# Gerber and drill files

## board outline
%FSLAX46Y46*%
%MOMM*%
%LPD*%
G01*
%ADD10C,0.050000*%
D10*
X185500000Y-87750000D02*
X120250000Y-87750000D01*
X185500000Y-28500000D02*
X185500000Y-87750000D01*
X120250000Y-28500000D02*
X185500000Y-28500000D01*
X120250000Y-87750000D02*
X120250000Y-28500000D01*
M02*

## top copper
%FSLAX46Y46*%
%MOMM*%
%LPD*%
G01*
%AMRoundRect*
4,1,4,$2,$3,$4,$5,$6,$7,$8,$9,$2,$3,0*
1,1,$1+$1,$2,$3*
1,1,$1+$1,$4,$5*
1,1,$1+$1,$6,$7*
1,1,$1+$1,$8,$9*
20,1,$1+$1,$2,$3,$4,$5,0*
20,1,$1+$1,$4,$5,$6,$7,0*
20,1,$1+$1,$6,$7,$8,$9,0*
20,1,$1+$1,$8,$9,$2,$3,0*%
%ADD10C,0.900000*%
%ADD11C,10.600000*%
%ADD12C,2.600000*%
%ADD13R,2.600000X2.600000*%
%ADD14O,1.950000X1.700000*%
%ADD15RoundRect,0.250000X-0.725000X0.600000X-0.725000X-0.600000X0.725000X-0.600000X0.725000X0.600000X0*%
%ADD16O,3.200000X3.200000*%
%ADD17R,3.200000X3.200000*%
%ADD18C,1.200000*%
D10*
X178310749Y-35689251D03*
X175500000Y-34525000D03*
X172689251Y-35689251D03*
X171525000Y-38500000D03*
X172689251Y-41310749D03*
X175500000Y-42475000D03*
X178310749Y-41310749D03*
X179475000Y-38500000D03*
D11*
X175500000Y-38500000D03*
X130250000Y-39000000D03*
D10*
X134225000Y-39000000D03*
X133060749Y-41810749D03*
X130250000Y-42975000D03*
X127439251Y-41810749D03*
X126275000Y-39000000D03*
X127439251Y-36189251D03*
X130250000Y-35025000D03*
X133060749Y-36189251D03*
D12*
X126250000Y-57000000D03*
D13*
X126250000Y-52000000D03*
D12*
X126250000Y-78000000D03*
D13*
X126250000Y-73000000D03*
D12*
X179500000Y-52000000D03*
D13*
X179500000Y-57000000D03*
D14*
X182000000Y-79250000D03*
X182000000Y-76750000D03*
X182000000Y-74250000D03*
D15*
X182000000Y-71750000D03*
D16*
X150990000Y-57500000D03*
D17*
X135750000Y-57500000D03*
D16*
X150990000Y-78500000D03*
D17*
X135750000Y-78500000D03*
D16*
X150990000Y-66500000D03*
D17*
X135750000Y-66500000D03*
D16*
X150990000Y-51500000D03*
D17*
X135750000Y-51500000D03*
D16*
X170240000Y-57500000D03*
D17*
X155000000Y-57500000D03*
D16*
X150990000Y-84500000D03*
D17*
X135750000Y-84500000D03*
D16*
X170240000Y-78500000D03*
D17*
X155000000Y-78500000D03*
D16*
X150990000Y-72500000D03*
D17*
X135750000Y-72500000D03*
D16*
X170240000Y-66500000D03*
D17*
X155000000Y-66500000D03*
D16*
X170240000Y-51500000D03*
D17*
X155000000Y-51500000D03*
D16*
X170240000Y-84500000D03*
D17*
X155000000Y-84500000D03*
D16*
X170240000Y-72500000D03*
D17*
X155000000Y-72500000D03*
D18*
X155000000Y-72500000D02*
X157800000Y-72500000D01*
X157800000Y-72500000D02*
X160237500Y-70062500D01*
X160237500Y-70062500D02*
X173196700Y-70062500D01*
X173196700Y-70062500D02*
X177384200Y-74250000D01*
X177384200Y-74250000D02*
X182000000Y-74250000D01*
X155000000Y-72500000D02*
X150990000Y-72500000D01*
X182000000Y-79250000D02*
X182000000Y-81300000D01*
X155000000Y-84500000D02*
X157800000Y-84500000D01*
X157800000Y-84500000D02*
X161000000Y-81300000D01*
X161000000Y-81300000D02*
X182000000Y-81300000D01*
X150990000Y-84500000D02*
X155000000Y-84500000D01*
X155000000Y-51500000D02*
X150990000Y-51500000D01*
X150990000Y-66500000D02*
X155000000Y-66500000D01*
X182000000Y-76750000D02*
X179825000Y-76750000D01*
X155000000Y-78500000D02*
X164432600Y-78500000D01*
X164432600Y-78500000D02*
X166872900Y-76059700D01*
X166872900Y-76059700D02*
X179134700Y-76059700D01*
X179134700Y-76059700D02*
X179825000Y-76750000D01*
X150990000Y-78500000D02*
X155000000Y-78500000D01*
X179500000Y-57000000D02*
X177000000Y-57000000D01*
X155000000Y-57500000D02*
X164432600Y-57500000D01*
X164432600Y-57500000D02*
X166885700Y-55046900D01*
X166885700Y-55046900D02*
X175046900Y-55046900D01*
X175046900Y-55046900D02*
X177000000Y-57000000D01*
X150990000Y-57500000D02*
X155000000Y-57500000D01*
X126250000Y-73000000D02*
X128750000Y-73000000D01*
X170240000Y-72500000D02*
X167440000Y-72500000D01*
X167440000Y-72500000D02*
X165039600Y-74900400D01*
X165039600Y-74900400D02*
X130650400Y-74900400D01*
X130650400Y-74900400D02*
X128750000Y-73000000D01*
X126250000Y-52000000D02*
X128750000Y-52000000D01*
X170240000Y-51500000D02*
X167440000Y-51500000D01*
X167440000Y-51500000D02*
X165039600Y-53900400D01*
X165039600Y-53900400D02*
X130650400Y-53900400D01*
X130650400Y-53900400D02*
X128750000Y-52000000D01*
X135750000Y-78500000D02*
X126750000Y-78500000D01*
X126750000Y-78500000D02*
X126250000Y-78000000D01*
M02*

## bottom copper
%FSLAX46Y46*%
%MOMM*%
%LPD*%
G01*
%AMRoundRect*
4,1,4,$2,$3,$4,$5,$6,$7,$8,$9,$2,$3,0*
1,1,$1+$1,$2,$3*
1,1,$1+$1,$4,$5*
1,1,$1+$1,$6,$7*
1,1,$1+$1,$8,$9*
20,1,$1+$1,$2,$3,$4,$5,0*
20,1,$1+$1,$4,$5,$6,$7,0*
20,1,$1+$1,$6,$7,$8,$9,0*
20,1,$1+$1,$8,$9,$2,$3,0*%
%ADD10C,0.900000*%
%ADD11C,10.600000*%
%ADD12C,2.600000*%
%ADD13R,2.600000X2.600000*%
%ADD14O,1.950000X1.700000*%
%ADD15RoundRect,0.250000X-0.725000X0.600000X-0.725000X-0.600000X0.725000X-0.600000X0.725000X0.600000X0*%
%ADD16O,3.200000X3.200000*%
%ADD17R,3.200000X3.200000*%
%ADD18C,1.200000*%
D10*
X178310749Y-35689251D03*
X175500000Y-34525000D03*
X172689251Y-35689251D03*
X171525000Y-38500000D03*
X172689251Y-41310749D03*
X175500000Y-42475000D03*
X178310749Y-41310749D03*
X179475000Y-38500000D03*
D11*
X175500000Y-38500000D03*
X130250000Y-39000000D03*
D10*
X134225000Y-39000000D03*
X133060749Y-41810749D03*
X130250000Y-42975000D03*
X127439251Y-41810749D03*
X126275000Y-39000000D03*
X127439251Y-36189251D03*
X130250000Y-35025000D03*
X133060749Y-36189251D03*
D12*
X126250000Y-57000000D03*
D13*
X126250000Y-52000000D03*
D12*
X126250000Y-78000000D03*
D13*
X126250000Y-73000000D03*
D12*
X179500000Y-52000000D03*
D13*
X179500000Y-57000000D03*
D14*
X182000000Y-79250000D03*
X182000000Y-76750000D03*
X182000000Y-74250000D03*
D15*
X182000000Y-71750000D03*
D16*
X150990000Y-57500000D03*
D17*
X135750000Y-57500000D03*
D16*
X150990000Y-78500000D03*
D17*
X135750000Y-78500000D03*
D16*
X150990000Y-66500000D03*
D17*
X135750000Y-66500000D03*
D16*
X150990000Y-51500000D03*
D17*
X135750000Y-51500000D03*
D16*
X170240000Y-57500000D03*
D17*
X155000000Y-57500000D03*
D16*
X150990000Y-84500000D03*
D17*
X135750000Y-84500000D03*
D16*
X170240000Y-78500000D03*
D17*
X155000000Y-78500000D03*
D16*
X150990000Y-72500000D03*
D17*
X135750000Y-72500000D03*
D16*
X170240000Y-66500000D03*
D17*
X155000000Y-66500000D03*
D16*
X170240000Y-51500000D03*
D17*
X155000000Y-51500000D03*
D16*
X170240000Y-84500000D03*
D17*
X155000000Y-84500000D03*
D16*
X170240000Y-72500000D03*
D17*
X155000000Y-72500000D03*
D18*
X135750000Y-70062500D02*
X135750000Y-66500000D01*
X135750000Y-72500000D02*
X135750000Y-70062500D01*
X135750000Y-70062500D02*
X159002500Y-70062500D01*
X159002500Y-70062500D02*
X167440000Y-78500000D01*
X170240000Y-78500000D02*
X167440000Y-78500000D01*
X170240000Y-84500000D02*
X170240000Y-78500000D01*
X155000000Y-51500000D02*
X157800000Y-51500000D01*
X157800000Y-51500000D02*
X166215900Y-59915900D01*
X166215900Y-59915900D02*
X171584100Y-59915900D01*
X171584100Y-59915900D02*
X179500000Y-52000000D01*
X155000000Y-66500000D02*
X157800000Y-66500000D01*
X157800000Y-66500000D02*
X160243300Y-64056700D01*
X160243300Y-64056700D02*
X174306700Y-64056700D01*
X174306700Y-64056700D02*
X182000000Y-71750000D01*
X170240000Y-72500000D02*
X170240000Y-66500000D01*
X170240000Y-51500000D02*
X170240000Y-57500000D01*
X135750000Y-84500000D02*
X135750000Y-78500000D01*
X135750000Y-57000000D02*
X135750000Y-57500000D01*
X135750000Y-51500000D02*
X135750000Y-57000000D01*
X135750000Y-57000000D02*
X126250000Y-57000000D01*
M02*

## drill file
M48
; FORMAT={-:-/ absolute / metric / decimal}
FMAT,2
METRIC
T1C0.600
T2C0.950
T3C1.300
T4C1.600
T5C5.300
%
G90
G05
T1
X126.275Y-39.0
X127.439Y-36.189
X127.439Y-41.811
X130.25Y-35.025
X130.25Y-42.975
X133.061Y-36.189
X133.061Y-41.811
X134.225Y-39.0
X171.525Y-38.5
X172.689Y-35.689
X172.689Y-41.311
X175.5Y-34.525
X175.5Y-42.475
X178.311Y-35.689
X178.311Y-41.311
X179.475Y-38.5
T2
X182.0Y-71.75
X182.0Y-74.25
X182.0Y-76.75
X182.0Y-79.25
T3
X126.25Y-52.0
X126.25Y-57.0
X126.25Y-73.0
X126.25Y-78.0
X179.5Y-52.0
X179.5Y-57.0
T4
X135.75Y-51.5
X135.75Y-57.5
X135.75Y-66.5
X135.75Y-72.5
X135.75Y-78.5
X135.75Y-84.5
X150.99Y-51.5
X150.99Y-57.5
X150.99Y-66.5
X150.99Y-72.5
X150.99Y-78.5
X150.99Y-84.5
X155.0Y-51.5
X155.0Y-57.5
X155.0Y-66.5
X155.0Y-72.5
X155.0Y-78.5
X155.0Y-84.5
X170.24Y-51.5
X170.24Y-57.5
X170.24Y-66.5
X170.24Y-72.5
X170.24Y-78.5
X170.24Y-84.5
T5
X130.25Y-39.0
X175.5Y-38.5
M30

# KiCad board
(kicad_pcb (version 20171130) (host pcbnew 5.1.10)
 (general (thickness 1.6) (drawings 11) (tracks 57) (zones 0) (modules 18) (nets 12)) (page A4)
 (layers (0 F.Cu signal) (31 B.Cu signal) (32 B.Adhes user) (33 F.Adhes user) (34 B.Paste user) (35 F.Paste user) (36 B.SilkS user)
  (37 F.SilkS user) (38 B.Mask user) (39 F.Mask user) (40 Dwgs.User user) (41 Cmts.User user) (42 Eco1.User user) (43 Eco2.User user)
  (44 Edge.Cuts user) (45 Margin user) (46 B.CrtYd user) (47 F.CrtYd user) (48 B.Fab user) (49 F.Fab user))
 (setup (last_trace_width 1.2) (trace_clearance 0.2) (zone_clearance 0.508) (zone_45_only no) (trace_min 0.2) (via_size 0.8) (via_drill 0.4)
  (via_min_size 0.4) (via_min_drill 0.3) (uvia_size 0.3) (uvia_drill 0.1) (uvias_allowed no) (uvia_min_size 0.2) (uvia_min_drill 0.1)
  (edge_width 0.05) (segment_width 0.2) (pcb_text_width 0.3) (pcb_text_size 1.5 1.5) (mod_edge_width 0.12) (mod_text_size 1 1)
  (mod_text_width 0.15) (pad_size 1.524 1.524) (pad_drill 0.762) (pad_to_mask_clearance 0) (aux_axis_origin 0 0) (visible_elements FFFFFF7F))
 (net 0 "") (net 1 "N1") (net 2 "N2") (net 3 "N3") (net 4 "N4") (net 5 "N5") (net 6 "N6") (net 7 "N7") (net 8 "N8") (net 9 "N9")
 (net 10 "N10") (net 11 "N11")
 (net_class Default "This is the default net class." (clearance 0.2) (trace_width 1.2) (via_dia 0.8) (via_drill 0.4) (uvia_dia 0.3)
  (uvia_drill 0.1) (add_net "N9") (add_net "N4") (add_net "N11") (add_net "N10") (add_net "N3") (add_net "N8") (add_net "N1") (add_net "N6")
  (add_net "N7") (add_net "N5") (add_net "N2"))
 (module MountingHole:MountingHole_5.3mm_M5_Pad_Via (layer F.Cu) (at 175.5 38.5)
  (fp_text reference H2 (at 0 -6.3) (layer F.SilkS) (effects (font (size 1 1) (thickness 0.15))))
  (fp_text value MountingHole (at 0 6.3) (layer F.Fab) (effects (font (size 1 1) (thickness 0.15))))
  (pad 1 thru_hole circle (at 2.810749 -2.810749) (size 0.9 0.9) (drill 0.6) (layers *.Cu *.Mask))
  (pad 1 thru_hole circle (at 0 -3.975) (size 0.9 0.9) (drill 0.6) (layers *.Cu *.Mask))
  (pad 1 thru_hole circle (at -2.810749 -2.810749) (size 0.9 0.9) (drill 0.6) (layers *.Cu *.Mask))
  (pad 1 thru_hole circle (at -3.975 0) (size 0.9 0.9) (drill 0.6) (layers *.Cu *.Mask))
  (pad 1 thru_hole circle (at -2.810749 2.810749) (size 0.9 0.9) (drill 0.6) (layers *.Cu *.Mask))
  (pad 1 thru_hole circle (at 0 3.975) (size 0.9 0.9) (drill 0.6) (layers *.Cu *.Mask))
  (pad 1 thru_hole circle (at 2.810749 2.810749) (size 0.9 0.9) (drill 0.6) (layers *.Cu *.Mask))
  (pad 1 thru_hole circle (at 3.975 0) (size 0.9 0.9) (drill 0.6) (layers *.Cu *.Mask))
  (pad 1 thru_hole circle (at 0 0) (size 10.6 10.6) (drill 5.3) (layers *.Cu *.Mask)))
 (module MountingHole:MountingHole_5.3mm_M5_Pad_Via (layer F.Cu) (at 130.25 39)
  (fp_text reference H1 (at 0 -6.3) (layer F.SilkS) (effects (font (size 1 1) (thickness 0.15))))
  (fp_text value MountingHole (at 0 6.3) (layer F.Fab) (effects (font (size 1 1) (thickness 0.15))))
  (pad 1 thru_hole circle (at 0 0) (size 10.6 10.6) (drill 5.3) (layers *.Cu *.Mask))
  (pad 1 thru_hole circle (at 3.975 0) (size 0.9 0.9) (drill 0.6) (layers *.Cu *.Mask))
  (pad 1 thru_hole circle (at 2.810749 2.810749) (size 0.9 0.9) (drill 0.6) (layers *.Cu *.Mask))
  (pad 1 thru_hole circle (at 0 3.975) (size 0.9 0.9) (drill 0.6) (layers *.Cu *.Mask))
  (pad 1 thru_hole circle (at -2.810749 2.810749) (size 0.9 0.9) (drill 0.6) (layers *.Cu *.Mask))
  (pad 1 thru_hole circle (at -3.975 0) (size 0.9 0.9) (drill 0.6) (layers *.Cu *.Mask))
  (pad 1 thru_hole circle (at -2.810749 -2.810749) (size 0.9 0.9) (drill 0.6) (layers *.Cu *.Mask))
  (pad 1 thru_hole circle (at 0 -3.975) (size 0.9 0.9) (drill 0.6) (layers *.Cu *.Mask))
  (pad 1 thru_hole circle (at 2.810749 -2.810749) (size 0.9 0.9) (drill 0.6) (layers *.Cu *.Mask)))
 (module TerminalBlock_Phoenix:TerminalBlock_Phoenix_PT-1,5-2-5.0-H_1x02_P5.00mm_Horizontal (layer F.Cu) (at 126.25 52 270)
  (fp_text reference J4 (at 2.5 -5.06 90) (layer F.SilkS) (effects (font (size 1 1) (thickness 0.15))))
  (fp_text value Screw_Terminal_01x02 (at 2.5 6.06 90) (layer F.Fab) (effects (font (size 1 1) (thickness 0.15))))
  (pad 2 thru_hole circle (at 5 0 270) (size 2.6 2.6) (drill 1.3) (layers *.Cu *.Mask) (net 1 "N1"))
  (pad 1 thru_hole rect (at 0 0 270) (size 2.6 2.6) (drill 1.3) (layers *.Cu *.Mask) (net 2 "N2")))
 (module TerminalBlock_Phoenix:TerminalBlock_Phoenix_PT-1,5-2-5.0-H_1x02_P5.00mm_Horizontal (layer F.Cu) (at 126.25 73 270)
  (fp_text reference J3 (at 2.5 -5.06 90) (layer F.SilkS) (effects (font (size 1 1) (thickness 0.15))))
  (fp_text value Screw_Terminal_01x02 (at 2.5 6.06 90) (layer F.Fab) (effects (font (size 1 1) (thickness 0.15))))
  (pad 2 thru_hole circle (at 5 0 270) (size 2.6 2.6) (drill 1.3) (layers *.Cu *.Mask) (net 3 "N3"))
  (pad 1 thru_hole rect (at 0 0 270) (size 2.6 2.6) (drill 1.3) (layers *.Cu *.Mask) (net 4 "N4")))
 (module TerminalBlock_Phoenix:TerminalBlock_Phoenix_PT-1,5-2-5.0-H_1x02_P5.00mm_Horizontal (layer F.Cu) (at 179.5 57 90)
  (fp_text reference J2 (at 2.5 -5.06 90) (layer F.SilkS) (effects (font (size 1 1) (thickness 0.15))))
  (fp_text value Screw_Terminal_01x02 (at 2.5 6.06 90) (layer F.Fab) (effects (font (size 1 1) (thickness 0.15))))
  (pad 2 thru_hole circle (at 5 0 90) (size 2.6 2.6) (drill 1.3) (layers *.Cu *.Mask) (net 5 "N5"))
  (pad 1 thru_hole rect (at 0 0 90) (size 2.6 2.6) (drill 1.3) (layers *.Cu *.Mask) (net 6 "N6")))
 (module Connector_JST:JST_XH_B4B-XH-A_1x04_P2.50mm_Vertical (layer F.Cu) (at 182 71.75 270)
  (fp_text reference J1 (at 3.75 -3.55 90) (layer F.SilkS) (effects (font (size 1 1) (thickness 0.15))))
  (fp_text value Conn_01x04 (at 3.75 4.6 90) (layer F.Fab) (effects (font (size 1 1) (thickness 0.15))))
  (pad 4 thru_hole oval (at 7.5 0 270) (size 1.7 1.95) (drill 0.95) (layers *.Cu *.Mask) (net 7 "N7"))
  (pad 3 thru_hole oval (at 5 0 270) (size 1.7 1.95) (drill 0.95) (layers *.Cu *.Mask) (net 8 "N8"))
  (pad 2 thru_hole oval (at 2.5 0 270) (size 1.7 1.95) (drill 0.95) (layers *.Cu *.Mask) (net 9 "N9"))
  (pad 1 thru_hole roundrect (at 0 0 270) (size 1.7 1.95) (drill 0.95) (layers *.Cu *.Mask) (roundrect_rratio 0.1470588235294118)
   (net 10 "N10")))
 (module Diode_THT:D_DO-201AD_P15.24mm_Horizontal (layer F.Cu) (at 135.75 57.5)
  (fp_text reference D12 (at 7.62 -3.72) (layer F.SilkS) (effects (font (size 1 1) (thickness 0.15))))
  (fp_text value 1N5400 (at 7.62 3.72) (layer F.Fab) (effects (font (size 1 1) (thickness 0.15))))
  (pad 2 thru_hole oval (at 15.24 0) (size 3.2 3.2) (drill 1.6) (layers *.Cu *.Mask) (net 6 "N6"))
  (pad 1 thru_hole rect (at 0 0) (size 3.2 3.2) (drill 1.6) (layers *.Cu *.Mask) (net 1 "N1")))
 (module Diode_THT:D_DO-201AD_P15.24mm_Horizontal (layer F.Cu) (at 135.75 78.5)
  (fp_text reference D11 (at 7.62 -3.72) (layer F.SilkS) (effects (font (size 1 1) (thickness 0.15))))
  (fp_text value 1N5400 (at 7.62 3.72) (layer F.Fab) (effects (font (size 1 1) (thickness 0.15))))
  (pad 2 thru_hole oval (at 15.24 0) (size 3.2 3.2) (drill 1.6) (layers *.Cu *.Mask) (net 8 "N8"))
  (pad 1 thru_hole rect (at 0 0) (size 3.2 3.2) (drill 1.6) (layers *.Cu *.Mask) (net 3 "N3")))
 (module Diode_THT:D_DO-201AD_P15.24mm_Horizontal (layer F.Cu) (at 135.75 66.5)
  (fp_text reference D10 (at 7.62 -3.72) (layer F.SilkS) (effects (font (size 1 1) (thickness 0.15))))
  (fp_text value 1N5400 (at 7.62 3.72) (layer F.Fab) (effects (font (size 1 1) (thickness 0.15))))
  (pad 2 thru_hole oval (at 15.24 0) (size 3.2 3.2) (drill 1.6) (layers *.Cu *.Mask) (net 10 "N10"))
  (pad 1 thru_hole rect (at 0 0) (size 3.2 3.2) (drill 1.6) (layers *.Cu *.Mask) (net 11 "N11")))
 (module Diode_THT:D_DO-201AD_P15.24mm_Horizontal (layer F.Cu) (at 135.75 51.5)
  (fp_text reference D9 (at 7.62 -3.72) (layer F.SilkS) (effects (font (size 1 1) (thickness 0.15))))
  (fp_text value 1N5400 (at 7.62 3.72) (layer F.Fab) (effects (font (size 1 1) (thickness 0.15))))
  (pad 2 thru_hole oval (at 15.24 0) (size 3.2 3.2) (drill 1.6) (layers *.Cu *.Mask) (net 5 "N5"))
  (pad 1 thru_hole rect (at 0 0) (size 3.2 3.2) (drill 1.6) (layers *.Cu *.Mask) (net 1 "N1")))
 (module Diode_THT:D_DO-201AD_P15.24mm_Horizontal (layer F.Cu) (at 155 57.5)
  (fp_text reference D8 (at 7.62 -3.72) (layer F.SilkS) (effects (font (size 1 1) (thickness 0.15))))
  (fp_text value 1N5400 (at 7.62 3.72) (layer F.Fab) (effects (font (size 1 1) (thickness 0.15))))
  (pad 2 thru_hole oval (at 15.24 0) (size 3.2 3.2) (drill 1.6) (layers *.Cu *.Mask) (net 2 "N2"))
  (pad 1 thru_hole rect (at 0 0) (size 3.2 3.2) (drill 1.6) (layers *.Cu *.Mask) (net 6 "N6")))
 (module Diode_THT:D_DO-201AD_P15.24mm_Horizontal (layer F.Cu) (at 135.75 84.5)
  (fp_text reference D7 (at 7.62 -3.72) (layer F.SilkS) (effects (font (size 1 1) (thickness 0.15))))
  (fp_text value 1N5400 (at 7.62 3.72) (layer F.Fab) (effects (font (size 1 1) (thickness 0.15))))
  (pad 2 thru_hole oval (at 15.24 0) (size 3.2 3.2) (drill 1.6) (layers *.Cu *.Mask) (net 7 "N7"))
  (pad 1 thru_hole rect (at 0 0) (size 3.2 3.2) (drill 1.6) (layers *.Cu *.Mask) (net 3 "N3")))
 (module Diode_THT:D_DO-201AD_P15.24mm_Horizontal (layer F.Cu) (at 155 78.5)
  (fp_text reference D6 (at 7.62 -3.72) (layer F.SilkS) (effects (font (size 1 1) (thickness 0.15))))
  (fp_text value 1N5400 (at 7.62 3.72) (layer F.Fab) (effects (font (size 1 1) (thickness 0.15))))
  (pad 2 thru_hole oval (at 15.24 0) (size 3.2 3.2) (drill 1.6) (layers *.Cu *.Mask) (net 11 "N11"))
  (pad 1 thru_hole rect (at 0 0) (size 3.2 3.2) (drill 1.6) (layers *.Cu *.Mask) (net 8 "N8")))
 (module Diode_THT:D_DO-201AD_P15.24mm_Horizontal (layer F.Cu) (at 135.75 72.5)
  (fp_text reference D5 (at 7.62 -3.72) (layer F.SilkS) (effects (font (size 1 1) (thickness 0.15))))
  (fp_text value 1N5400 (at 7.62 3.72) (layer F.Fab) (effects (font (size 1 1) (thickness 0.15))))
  (pad 2 thru_hole oval (at 15.24 0) (size 3.2 3.2) (drill 1.6) (layers *.Cu *.Mask) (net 9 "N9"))
  (pad 1 thru_hole rect (at 0 0) (size 3.2 3.2) (drill 1.6) (layers *.Cu *.Mask) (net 11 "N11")))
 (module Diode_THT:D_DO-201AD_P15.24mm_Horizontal (layer F.Cu) (at 155 66.5)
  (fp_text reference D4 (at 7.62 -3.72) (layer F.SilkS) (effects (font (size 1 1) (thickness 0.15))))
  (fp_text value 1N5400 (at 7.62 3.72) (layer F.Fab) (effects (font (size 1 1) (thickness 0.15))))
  (pad 2 thru_hole oval (at 15.24 0) (size 3.2 3.2) (drill 1.6) (layers *.Cu *.Mask) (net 4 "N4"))
  (pad 1 thru_hole rect (at 0 0) (size 3.2 3.2) (drill 1.6) (layers *.Cu *.Mask) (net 10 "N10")))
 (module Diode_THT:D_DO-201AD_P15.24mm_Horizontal (layer F.Cu) (at 155 51.5)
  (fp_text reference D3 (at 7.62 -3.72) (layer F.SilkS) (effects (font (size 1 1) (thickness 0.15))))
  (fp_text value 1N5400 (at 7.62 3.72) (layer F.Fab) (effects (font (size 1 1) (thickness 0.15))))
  (pad 2 thru_hole oval (at 15.24 0) (size 3.2 3.2) (drill 1.6) (layers *.Cu *.Mask) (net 2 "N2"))
  (pad 1 thru_hole rect (at 0 0) (size 3.2 3.2) (drill 1.6) (layers *.Cu *.Mask) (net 5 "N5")))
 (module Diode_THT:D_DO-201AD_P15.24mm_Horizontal (layer F.Cu) (at 155 84.5)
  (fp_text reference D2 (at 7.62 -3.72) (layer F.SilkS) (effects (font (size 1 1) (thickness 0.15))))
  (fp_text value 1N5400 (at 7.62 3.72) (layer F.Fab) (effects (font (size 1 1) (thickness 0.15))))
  (pad 2 thru_hole oval (at 15.24 0) (size 3.2 3.2) (drill 1.6) (layers *.Cu *.Mask) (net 11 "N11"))
  (pad 1 thru_hole rect (at 0 0) (size 3.2 3.2) (drill 1.6) (layers *.Cu *.Mask) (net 7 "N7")))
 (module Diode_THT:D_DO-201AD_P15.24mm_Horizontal (layer F.Cu) (at 155 72.5)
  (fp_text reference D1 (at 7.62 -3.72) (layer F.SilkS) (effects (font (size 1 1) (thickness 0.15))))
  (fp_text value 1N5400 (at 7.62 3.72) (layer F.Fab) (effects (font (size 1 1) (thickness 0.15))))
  (pad 2 thru_hole oval (at 15.24 0) (size 3.2 3.2) (drill 1.6) (layers *.Cu *.Mask) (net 4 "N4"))
  (pad 1 thru_hole rect (at 0 0) (size 3.2 3.2) (drill 1.6) (layers *.Cu *.Mask) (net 9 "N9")))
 (gr_line (start 185.5 87.75) (end 120.25 87.75) (layer Edge.Cuts) (width 0.05))
 (gr_line (start 185.5 28.5) (end 185.5 87.75) (layer Edge.Cuts) (width 0.05))
 (gr_line (start 120.25 28.5) (end 185.5 28.5) (layer Edge.Cuts) (width 0.05))
 (gr_line (start 120.25 87.75) (end 120.25 28.5) (layer Edge.Cuts) (width 0.05))
 (segment (start 155 72.5) (end 157.8 72.5) (width 1.2) (layer F.Cu) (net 9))
 (segment (start 157.8 72.5) (end 160.2375 70.0625) (width 1.2) (layer F.Cu) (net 9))
 (segment (start 160.2375 70.0625) (end 173.1967 70.0625) (width 1.2) (layer F.Cu) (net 9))
 (segment (start 173.1967 70.0625) (end 177.3842 74.25) (width 1.2) (layer F.Cu) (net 9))
 (segment (start 177.3842 74.25) (end 182 74.25) (width 1.2) (layer F.Cu) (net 9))
 (segment (start 155 72.5) (end 150.99 72.5) (width 1.2) (layer F.Cu) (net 9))
 (segment (start 135.75 70.0625) (end 135.75 66.5) (width 1.2) (layer B.Cu) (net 11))
 (segment (start 135.75 72.5) (end 135.75 70.0625) (width 1.2) (layer B.Cu) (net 11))
 (segment (start 135.75 70.0625) (end 159.0025 70.0625) (width 1.2) (layer B.Cu) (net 11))
 (segment (start 159.0025 70.0625) (end 167.44 78.5) (width 1.2) (layer B.Cu) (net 11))
 (segment (start 170.24 78.5) (end 167.44 78.5) (width 1.2) (layer B.Cu) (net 11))
 (segment (start 170.24 84.5) (end 170.24 78.5) (width 1.2) (layer B.Cu) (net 11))
 (segment (start 182 79.25) (end 182 81.3) (width 1.2) (layer F.Cu) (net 7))
 (segment (start 155 84.5) (end 157.8 84.5) (width 1.2) (layer F.Cu) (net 7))
 (segment (start 157.8 84.5) (end 161 81.3) (width 1.2) (layer F.Cu) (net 7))
 (segment (start 161 81.3) (end 182 81.3) (width 1.2) (layer F.Cu) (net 7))
 (segment (start 150.99 84.5) (end 155 84.5) (width 1.2) (layer F.Cu) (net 7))
 (segment (start 155 51.5) (end 157.8 51.5) (width 1.2) (layer B.Cu) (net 5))
 (segment (start 157.8 51.5) (end 166.2159 59.9159) (width 1.2) (layer B.Cu) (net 5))
 (segment (start 166.2159 59.9159) (end 171.5841 59.9159) (width 1.2) (layer B.Cu) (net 5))
 (segment (start 171.5841 59.9159) (end 179.5 52) (width 1.2) (layer B.Cu) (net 5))
 (segment (start 155 51.5) (end 150.99 51.5) (width 1.2) (layer F.Cu) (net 5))
 (segment (start 155 66.5) (end 157.8 66.5) (width 1.2) (layer B.Cu) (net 10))
 (segment (start 157.8 66.5) (end 160.2433 64.0567) (width 1.2) (layer B.Cu) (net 10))
 (segment (start 160.2433 64.0567) (end 174.3067 64.0567) (width 1.2) (layer B.Cu) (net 10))
 (segment (start 174.3067 64.0567) (end 182 71.75) (width 1.2) (layer B.Cu) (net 10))
 (segment (start 150.99 66.5) (end 155 66.5) (width 1.2) (layer F.Cu) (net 10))
 (segment (start 182 76.75) (end 179.825 76.75) (width 1.2) (layer F.Cu) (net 8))
 (segment (start 155 78.5) (end 164.4326 78.5) (width 1.2) (layer F.Cu) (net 8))
 (segment (start 164.4326 78.5) (end 166.8729 76.0597) (width 1.2) (layer F.Cu) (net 8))
 (segment (start 166.8729 76.0597) (end 179.1347 76.0597) (width 1.2) (layer F.Cu) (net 8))
 (segment (start 179.1347 76.0597) (end 179.825 76.75) (width 1.2) (layer F.Cu) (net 8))
 (segment (start 150.99 78.5) (end 155 78.5) (width 1.2) (layer F.Cu) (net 8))
 (segment (start 179.5 57) (end 177 57) (width 1.2) (layer F.Cu) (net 6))
 (segment (start 155 57.5) (end 164.4326 57.5) (width 1.2) (layer F.Cu) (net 6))
 (segment (start 164.4326 57.5) (end 166.8857 55.0469) (width 1.2) (layer F.Cu) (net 6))
 (segment (start 166.8857 55.0469) (end 175.0469 55.0469) (width 1.2) (layer F.Cu) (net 6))
 (segment (start 175.0469 55.0469) (end 177 57) (width 1.2) (layer F.Cu) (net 6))
 (segment (start 150.99 57.5) (end 155 57.5) (width 1.2) (layer F.Cu) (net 6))
 (segment (start 126.25 73) (end 128.75 73) (width 1.2) (layer F.Cu) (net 4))
 (segment (start 170.24 72.5) (end 167.44 72.5) (width 1.2) (layer F.Cu) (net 4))
 (segment (start 167.44 72.5) (end 165.0396 74.9004) (width 1.2) (layer F.Cu) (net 4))
 (segment (start 165.0396 74.9004) (end 130.6504 74.9004) (width 1.2) (layer F.Cu) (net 4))
 (segment (start 130.6504 74.9004) (end 128.75 73) (width 1.2) (layer F.Cu) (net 4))
 (segment (start 170.24 72.5) (end 170.24 66.5) (width 1.2) (layer B.Cu) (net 4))
 (segment (start 126.25 52) (end 128.75 52) (width 1.2) (layer F.Cu) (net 2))
 (segment (start 170.24 51.5) (end 167.44 51.5) (width 1.2) (layer F.Cu) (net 2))
 (segment (start 167.44 51.5) (end 165.0396 53.9004) (width 1.2) (layer F.Cu) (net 2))
 (segment (start 165.0396 53.9004) (end 130.6504 53.9004) (width 1.2) (layer F.Cu) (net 2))
 (segment (start 130.6504 53.9004) (end 128.75 52) (width 1.2) (layer F.Cu) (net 2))
 (segment (start 170.24 51.5) (end 170.24 57.5) (width 1.2) (layer B.Cu) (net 2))
 (segment (start 135.75 78.5) (end 126.75 78.5) (width 1.2) (layer F.Cu) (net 3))
 (segment (start 126.75 78.5) (end 126.25 78) (width 1.2) (layer F.Cu) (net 3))
 (segment (start 135.75 84.5) (end 135.75 78.5) (width 1.2) (layer B.Cu) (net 3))
 (segment (start 135.75 57) (end 135.75 57.5) (width 1.2) (layer B.Cu) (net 1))
 (segment (start 135.75 51.5) (end 135.75 57) (width 1.2) (layer B.Cu) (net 1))
 (segment (start 135.75 57) (end 126.25 57) (width 1.2) (layer B.Cu) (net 1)))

